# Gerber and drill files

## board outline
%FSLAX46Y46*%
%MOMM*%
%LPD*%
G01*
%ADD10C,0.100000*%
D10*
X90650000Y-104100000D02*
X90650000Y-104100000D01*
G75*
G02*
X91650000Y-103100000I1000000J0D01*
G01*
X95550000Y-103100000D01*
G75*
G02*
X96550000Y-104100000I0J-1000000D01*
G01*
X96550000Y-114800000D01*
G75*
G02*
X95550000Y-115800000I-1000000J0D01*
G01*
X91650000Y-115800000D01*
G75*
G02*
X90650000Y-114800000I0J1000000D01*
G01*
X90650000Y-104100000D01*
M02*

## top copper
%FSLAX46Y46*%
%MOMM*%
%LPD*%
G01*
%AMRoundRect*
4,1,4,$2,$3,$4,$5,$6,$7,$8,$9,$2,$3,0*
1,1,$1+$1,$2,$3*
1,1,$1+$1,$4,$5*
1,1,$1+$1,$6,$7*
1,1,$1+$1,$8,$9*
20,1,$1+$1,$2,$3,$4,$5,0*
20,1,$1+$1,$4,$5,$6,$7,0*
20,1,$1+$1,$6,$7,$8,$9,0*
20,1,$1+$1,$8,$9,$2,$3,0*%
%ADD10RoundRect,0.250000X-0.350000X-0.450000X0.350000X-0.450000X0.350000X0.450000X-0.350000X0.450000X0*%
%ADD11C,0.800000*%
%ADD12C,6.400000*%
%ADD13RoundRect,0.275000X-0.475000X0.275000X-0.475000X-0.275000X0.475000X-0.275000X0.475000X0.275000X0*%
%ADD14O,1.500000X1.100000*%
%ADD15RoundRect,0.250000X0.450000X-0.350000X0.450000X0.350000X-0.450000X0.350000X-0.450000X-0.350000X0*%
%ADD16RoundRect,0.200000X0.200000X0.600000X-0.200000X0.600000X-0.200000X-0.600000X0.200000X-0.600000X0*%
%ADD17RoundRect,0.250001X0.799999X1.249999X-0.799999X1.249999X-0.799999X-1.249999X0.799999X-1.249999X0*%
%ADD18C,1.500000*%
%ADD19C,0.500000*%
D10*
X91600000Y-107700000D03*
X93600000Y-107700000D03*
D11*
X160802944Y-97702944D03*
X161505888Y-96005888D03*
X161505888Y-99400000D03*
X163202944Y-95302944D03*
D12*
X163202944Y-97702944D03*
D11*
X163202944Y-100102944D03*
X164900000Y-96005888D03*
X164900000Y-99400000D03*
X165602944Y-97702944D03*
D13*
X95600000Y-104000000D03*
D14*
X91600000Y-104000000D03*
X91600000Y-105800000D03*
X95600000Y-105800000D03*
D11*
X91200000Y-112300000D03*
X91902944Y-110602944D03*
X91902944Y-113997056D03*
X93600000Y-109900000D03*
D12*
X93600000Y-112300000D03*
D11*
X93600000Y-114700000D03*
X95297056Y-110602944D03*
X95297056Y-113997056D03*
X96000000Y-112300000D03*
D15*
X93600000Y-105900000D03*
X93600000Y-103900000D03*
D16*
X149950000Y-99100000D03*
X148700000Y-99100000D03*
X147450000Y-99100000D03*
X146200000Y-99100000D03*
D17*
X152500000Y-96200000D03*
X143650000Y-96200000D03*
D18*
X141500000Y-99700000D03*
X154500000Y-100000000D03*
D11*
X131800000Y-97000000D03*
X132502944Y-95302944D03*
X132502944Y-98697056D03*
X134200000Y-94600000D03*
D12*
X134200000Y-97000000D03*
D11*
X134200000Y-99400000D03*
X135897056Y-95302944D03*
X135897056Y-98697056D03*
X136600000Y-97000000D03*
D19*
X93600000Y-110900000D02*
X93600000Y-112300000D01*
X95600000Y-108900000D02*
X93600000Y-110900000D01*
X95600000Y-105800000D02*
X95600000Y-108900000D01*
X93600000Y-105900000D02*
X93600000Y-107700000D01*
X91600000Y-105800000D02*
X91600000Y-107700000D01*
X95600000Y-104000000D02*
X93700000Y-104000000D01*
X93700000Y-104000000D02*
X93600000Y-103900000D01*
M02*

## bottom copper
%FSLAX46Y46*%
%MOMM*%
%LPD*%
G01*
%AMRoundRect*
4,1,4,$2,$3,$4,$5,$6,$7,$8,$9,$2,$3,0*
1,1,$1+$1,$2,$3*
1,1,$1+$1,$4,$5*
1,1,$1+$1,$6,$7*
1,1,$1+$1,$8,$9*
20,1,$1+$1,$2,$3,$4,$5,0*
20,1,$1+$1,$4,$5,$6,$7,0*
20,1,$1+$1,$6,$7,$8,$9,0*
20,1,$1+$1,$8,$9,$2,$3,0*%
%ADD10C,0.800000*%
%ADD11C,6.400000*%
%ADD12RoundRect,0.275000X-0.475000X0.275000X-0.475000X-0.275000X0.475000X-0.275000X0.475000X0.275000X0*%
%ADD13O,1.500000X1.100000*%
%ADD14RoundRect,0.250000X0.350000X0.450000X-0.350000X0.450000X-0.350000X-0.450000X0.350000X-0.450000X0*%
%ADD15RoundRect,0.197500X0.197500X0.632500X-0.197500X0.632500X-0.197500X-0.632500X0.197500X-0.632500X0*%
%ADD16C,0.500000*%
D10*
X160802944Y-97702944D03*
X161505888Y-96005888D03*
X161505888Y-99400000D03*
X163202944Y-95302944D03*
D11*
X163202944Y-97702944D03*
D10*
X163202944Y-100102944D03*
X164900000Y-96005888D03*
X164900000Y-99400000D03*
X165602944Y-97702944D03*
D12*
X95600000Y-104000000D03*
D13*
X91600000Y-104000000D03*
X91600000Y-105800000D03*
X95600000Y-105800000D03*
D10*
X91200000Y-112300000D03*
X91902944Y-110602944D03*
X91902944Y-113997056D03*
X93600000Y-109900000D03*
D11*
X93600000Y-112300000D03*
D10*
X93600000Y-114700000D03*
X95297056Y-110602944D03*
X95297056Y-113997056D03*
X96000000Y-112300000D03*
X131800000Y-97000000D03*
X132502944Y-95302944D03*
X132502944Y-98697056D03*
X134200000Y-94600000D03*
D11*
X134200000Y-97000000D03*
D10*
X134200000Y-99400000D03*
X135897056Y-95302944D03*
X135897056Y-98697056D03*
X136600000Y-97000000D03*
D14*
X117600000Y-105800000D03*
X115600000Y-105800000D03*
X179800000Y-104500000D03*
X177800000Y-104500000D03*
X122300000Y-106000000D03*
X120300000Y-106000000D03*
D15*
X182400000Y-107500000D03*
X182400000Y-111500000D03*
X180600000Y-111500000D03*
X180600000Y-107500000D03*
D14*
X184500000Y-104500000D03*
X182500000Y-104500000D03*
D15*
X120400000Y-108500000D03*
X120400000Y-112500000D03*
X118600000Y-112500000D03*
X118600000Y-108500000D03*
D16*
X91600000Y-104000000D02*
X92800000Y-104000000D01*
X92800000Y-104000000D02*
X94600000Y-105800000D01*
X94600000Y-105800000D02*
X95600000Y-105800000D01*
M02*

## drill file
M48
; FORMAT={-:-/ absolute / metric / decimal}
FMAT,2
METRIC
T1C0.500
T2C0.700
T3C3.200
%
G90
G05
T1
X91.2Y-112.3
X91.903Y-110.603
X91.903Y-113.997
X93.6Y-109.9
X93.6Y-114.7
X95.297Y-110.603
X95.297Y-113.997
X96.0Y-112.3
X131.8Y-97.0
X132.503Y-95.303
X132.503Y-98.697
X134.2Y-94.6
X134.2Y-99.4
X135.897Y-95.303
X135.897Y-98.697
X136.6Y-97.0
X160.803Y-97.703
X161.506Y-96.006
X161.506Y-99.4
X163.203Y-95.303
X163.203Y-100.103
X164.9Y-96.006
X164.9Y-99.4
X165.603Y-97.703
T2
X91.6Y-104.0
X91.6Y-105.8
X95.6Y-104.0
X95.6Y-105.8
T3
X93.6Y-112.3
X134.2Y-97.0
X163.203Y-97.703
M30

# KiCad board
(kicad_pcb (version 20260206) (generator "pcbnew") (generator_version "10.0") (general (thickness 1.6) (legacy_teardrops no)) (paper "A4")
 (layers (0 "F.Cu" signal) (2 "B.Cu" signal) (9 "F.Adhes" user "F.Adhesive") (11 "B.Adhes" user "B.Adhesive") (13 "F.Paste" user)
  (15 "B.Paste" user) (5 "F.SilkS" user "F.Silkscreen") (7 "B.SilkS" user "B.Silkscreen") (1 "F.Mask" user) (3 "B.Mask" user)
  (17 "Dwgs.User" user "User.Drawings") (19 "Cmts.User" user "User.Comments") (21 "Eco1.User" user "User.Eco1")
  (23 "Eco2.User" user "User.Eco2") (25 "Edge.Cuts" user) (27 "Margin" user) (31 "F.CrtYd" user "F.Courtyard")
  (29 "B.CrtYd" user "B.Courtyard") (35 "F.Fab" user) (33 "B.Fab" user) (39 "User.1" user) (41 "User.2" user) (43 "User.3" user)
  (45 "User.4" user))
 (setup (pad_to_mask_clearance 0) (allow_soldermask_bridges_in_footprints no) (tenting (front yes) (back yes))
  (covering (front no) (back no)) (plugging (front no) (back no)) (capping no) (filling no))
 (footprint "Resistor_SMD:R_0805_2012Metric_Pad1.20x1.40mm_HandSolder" (layer "F.Cu") (at 92.6 107.7)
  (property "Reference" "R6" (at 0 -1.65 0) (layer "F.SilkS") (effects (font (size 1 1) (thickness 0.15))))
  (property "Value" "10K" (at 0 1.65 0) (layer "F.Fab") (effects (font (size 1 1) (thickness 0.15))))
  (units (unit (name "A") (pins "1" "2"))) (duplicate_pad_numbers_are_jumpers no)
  (pad "1" smd roundrect (at -1 0) (size 1.2 1.4) (layers "F.Cu" "F.Mask" "F.Paste") (roundrect_rratio 0.208333) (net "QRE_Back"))
  (pad "2" smd roundrect (at 1 0) (size 1.2 1.4) (layers "F.Cu" "F.Mask" "F.Paste") (roundrect_rratio 0.208333) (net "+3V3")))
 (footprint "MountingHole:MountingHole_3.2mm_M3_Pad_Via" (layer "F.Cu") (at 163.202944 97.702944)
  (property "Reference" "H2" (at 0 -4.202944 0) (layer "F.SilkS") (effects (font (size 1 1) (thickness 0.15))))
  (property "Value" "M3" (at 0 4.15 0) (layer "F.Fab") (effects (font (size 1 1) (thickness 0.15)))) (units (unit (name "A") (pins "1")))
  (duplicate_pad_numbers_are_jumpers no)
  (pad "1" thru_hole circle (at -2.4 0) (size 0.8 0.8) (drill 0.5) (layers "*.Cu" "*.Mask") (remove_unused_layers no) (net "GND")
   (zone_connect 2))
  (pad "1" thru_hole circle (at -1.697056 -1.697056) (size 0.8 0.8) (drill 0.5) (layers "*.Cu" "*.Mask") (remove_unused_layers no)
   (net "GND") (zone_connect 2))
  (pad "1" thru_hole circle (at -1.697056 1.697056) (size 0.8 0.8) (drill 0.5) (layers "*.Cu" "*.Mask") (remove_unused_layers no)
   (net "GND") (zone_connect 2))
  (pad "1" thru_hole circle (at 0 -2.4) (size 0.8 0.8) (drill 0.5) (layers "*.Cu" "*.Mask") (remove_unused_layers no) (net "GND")
   (zone_connect 2))
  (pad "1" thru_hole circle (at 0 0) (size 6.4 6.4) (drill 3.2) (layers "*.Cu" "*.Mask") (remove_unused_layers no) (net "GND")
   (zone_connect 2))
  (pad "1" thru_hole circle (at 0 2.4) (size 0.8 0.8) (drill 0.5) (layers "*.Cu" "*.Mask") (remove_unused_layers no) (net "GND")
   (zone_connect 2))
  (pad "1" thru_hole circle (at 1.697056 -1.697056) (size 0.8 0.8) (drill 0.5) (layers "*.Cu" "*.Mask") (remove_unused_layers no)
   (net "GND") (zone_connect 2))
  (pad "1" thru_hole circle (at 1.697056 1.697056) (size 0.8 0.8) (drill 0.5) (layers "*.Cu" "*.Mask") (remove_unused_layers no) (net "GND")
   (zone_connect 2))
  (pad "1" thru_hole circle (at 2.4 0) (size 0.8 0.8) (drill 0.5) (layers "*.Cu" "*.Mask") (remove_unused_layers no) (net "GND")
   (zone_connect 2)))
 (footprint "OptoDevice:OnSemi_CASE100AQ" (layer "F.Cu") (at 95.6 104 -90)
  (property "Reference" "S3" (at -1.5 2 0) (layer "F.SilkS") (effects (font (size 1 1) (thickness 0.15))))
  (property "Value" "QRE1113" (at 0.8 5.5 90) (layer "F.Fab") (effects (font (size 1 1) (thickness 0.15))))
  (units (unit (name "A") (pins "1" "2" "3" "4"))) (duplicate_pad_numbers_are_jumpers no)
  (pad "1" thru_hole roundrect (at 0 0 270) (size 1.1 1.5) (drill 0.7) (layers "*.Cu" "*.Mask") (remove_unused_layers no)
   (roundrect_rratio 0.25) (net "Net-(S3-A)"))
  (pad "2" thru_hole oval (at 0 4 270) (size 1.1 1.5) (drill 0.7) (layers "*.Cu" "*.Mask") (remove_unused_layers no) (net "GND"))
  (pad "3" thru_hole oval (at 1.8 4 270) (size 1.1 1.5) (drill 0.7) (layers "*.Cu" "*.Mask") (remove_unused_layers no) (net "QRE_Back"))
  (pad "4" thru_hole oval (at 1.8 0 270) (size 1.1 1.5) (drill 0.7) (layers "*.Cu" "*.Mask") (remove_unused_layers no) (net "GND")))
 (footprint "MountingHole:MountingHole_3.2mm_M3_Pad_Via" (layer "F.Cu") (at 93.6 112.3)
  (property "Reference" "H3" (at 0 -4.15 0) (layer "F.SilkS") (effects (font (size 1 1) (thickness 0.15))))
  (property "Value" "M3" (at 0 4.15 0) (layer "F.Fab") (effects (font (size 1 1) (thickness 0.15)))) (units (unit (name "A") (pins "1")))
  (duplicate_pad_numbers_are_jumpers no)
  (pad "1" thru_hole circle (at -2.4 0) (size 0.8 0.8) (drill 0.5) (layers "*.Cu" "*.Mask") (remove_unused_layers no) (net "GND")
   (zone_connect 2))
  (pad "1" thru_hole circle (at -1.697056 -1.697056) (size 0.8 0.8) (drill 0.5) (layers "*.Cu" "*.Mask") (remove_unused_layers no)
   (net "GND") (zone_connect 2))
  (pad "1" thru_hole circle (at -1.697056 1.697056) (size 0.8 0.8) (drill 0.5) (layers "*.Cu" "*.Mask") (remove_unused_layers no)
   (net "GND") (zone_connect 2))
  (pad "1" thru_hole circle (at 0 -2.4) (size 0.8 0.8) (drill 0.5) (layers "*.Cu" "*.Mask") (remove_unused_layers no) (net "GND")
   (zone_connect 2))
  (pad "1" thru_hole circle (at 0 0) (size 6.4 6.4) (drill 3.2) (layers "*.Cu" "*.Mask") (remove_unused_layers no) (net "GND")
   (zone_connect 2))
  (pad "1" thru_hole circle (at 0 2.4) (size 0.8 0.8) (drill 0.5) (layers "*.Cu" "*.Mask") (remove_unused_layers no) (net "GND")
   (zone_connect 2))
  (pad "1" thru_hole circle (at 1.697056 -1.697056) (size 0.8 0.8) (drill 0.5) (layers "*.Cu" "*.Mask") (remove_unused_layers no)
   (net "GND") (zone_connect 2))
  (pad "1" thru_hole circle (at 1.697056 1.697056) (size 0.8 0.8) (drill 0.5) (layers "*.Cu" "*.Mask") (remove_unused_layers no) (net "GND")
   (zone_connect 2))
  (pad "1" thru_hole circle (at 2.4 0) (size 0.8 0.8) (drill 0.5) (layers "*.Cu" "*.Mask") (remove_unused_layers no) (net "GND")
   (zone_connect 2)))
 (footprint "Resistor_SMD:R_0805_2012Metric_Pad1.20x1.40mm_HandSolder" (layer "F.Cu") (at 93.6 104.9 90)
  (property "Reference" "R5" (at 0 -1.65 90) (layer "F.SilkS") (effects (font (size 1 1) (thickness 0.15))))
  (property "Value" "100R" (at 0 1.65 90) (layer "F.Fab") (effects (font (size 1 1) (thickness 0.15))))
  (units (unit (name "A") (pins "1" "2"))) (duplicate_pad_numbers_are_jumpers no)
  (pad "1" smd roundrect (at -1 0 90) (size 1.2 1.4) (layers "F.Cu" "F.Mask" "F.Paste") (roundrect_rratio 0.208333) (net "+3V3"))
  (pad "2" smd roundrect (at 1 0 90) (size 1.2 1.4) (layers "F.Cu" "F.Mask" "F.Paste") (roundrect_rratio 0.208333) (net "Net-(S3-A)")))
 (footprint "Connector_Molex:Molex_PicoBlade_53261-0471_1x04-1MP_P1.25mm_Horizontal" (layer "F.Cu") (at 148.075 96.7 180)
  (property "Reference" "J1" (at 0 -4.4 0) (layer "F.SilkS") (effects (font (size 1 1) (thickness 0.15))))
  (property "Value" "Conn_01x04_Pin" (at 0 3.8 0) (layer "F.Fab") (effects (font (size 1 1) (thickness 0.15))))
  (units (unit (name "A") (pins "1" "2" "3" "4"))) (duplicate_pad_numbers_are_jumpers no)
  (pad "1" smd roundrect (at -1.875 -2.4 180) (size 0.8 1.6) (layers "F.Cu" "F.Mask" "F.Paste") (roundrect_rratio 0.25) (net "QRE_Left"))
  (pad "2" smd roundrect (at -0.625 -2.4 180) (size 0.8 1.6) (layers "F.Cu" "F.Mask" "F.Paste") (roundrect_rratio 0.25) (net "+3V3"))
  (pad "3" smd roundrect (at 0.625 -2.4 180) (size 0.8 1.6) (layers "F.Cu" "F.Mask" "F.Paste") (roundrect_rratio 0.25) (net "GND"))
  (pad "4" smd roundrect (at 1.875 -2.4 180) (size 0.8 1.6) (layers "F.Cu" "F.Mask" "F.Paste") (roundrect_rratio 0.25) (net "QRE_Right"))
  (pad "MP" smd roundrect (at -4.425 0.5 180) (size 2.1 3) (layers "F.Cu" "F.Mask" "F.Paste") (roundrect_rratio 0.119048))
  (pad "MP" smd roundrect (at 4.425 0.5 180) (size 2.1 3) (layers "F.Cu" "F.Mask" "F.Paste") (roundrect_rratio 0.119048)))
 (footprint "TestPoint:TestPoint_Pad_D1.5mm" (layer "F.Cu") (at 141.5 99.7)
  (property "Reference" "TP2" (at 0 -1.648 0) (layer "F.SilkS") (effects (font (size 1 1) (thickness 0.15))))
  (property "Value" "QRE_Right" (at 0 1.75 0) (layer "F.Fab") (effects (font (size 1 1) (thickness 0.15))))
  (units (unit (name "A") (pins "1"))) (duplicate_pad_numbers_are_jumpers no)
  (pad "1" smd circle (at 0 0) (size 1.5 1.5) (layers "F.Cu" "F.Mask") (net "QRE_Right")))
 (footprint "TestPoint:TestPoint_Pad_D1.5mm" (layer "F.Cu") (at 154.5 100)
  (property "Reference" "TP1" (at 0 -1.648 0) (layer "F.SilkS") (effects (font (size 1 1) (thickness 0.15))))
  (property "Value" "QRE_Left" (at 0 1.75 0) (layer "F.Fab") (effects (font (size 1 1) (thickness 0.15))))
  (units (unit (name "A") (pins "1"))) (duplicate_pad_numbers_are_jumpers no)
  (pad "1" smd circle (at 0 0) (size 1.5 1.5) (layers "F.Cu" "F.Mask") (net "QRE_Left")))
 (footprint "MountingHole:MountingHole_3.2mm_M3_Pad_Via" (layer "F.Cu") (at 134.2 97)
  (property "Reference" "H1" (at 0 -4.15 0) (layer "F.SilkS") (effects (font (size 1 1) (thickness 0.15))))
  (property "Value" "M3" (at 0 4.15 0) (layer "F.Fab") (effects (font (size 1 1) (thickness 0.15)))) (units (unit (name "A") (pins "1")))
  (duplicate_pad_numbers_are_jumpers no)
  (pad "1" thru_hole circle (at -2.4 0) (size 0.8 0.8) (drill 0.5) (layers "*.Cu" "*.Mask") (remove_unused_layers no) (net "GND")
   (zone_connect 2))
  (pad "1" thru_hole circle (at -1.697056 -1.697056) (size 0.8 0.8) (drill 0.5) (layers "*.Cu" "*.Mask") (remove_unused_layers no)
   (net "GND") (zone_connect 2))
  (pad "1" thru_hole circle (at -1.697056 1.697056) (size 0.8 0.8) (drill 0.5) (layers "*.Cu" "*.Mask") (remove_unused_layers no)
   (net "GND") (zone_connect 2))
  (pad "1" thru_hole circle (at 0 -2.4) (size 0.8 0.8) (drill 0.5) (layers "*.Cu" "*.Mask") (remove_unused_layers no) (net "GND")
   (zone_connect 2))
  (pad "1" thru_hole circle (at 0 0) (size 6.4 6.4) (drill 3.2) (layers "*.Cu" "*.Mask") (remove_unused_layers no) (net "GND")
   (zone_connect 2))
  (pad "1" thru_hole circle (at 0 2.4) (size 0.8 0.8) (drill 0.5) (layers "*.Cu" "*.Mask") (remove_unused_layers no) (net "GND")
   (zone_connect 2))
  (pad "1" thru_hole circle (at 1.697056 -1.697056) (size 0.8 0.8) (drill 0.5) (layers "*.Cu" "*.Mask") (remove_unused_layers no)
   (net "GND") (zone_connect 2))
  (pad "1" thru_hole circle (at 1.697056 1.697056) (size 0.8 0.8) (drill 0.5) (layers "*.Cu" "*.Mask") (remove_unused_layers no) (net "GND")
   (zone_connect 2))
  (pad "1" thru_hole circle (at 2.4 0) (size 0.8 0.8) (drill 0.5) (layers "*.Cu" "*.Mask") (remove_unused_layers no) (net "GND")
   (zone_connect 2)))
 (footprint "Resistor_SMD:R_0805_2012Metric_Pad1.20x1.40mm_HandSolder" (layer "B.Cu") (at 116.6 105.8 180)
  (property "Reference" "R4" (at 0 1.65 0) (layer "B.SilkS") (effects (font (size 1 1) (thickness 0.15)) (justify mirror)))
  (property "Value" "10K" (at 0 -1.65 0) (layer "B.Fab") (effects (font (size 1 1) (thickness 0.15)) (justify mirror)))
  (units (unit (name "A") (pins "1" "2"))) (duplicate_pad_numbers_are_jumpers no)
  (pad "1" smd roundrect (at -1 0 180) (size 1.2 1.4) (layers "B.Cu" "B.Mask" "B.Paste") (roundrect_rratio 0.208333) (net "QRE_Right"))
  (pad "2" smd roundrect (at 1 0 180) (size 1.2 1.4) (layers "B.Cu" "B.Mask" "B.Paste") (roundrect_rratio 0.208333) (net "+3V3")))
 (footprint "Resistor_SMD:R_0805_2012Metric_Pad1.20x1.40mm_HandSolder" (layer "B.Cu") (at 178.8 104.5 180)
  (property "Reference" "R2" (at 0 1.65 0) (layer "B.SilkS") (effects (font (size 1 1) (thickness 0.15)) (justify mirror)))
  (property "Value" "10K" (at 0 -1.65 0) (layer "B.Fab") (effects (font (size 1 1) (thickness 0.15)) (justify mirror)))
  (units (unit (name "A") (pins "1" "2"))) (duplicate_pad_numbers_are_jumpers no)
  (pad "1" smd roundrect (at -1 0 180) (size 1.2 1.4) (layers "B.Cu" "B.Mask" "B.Paste") (roundrect_rratio 0.208333) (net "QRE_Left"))
  (pad "2" smd roundrect (at 1 0 180) (size 1.2 1.4) (layers "B.Cu" "B.Mask" "B.Paste") (roundrect_rratio 0.208333) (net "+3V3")))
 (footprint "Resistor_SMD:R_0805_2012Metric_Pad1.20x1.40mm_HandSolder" (layer "B.Cu") (at 121.3 106 180)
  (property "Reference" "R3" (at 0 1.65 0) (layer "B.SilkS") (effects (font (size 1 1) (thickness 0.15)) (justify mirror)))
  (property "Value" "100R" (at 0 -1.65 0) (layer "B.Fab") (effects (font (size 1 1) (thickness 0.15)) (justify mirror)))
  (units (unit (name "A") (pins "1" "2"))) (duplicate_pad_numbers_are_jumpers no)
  (pad "1" smd roundrect (at -1 0 180) (size 1.2 1.4) (layers "B.Cu" "B.Mask" "B.Paste") (roundrect_rratio 0.208333) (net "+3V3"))
  (pad "2" smd roundrect (at 1 0 180) (size 1.2 1.4) (layers "B.Cu" "B.Mask" "B.Paste") (roundrect_rratio 0.208333) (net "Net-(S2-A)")))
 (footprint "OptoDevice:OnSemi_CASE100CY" (layer "B.Cu") (at 181.5 109.5 180)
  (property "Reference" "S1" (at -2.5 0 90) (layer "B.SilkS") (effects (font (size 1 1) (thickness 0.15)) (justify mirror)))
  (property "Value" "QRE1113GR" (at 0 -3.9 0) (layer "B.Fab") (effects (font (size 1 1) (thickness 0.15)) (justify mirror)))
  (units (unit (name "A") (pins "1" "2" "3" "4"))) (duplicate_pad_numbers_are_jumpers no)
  (pad "1" smd roundrect (at -0.9 2 180) (size 0.79 1.66) (layers "B.Cu" "B.Mask" "B.Paste") (roundrect_rratio 0.25) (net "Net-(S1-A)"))
  (pad "2" smd roundrect (at -0.9 -2 180) (size 0.79 1.66) (layers "B.Cu" "B.Mask" "B.Paste") (roundrect_rratio 0.25) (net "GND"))
  (pad "3" smd roundrect (at 0.9 -2 180) (size 0.79 1.66) (layers "B.Cu" "B.Mask" "B.Paste") (roundrect_rratio 0.25) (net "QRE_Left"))
  (pad "4" smd roundrect (at 0.9 2 180) (size 0.79 1.66) (layers "B.Cu" "B.Mask" "B.Paste") (roundrect_rratio 0.25) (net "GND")))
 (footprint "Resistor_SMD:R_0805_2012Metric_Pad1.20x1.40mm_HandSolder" (layer "B.Cu") (at 183.5 104.5 180)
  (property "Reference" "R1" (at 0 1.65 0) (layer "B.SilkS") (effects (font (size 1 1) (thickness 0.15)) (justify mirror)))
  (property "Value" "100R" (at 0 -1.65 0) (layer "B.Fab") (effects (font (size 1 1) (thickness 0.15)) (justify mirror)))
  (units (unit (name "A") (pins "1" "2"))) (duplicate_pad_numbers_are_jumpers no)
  (pad "1" smd roundrect (at -1 0 180) (size 1.2 1.4) (layers "B.Cu" "B.Mask" "B.Paste") (roundrect_rratio 0.208333) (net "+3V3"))
  (pad "2" smd roundrect (at 1 0 180) (size 1.2 1.4) (layers "B.Cu" "B.Mask" "B.Paste") (roundrect_rratio 0.208333) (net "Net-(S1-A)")))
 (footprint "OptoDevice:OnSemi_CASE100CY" (layer "B.Cu") (at 119.5 110.5 180)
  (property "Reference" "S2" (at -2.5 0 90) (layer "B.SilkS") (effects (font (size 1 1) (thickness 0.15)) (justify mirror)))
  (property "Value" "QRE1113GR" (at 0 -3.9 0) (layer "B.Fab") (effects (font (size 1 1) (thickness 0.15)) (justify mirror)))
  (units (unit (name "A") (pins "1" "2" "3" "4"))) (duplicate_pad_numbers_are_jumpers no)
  (pad "1" smd roundrect (at -0.9 2 180) (size 0.79 1.66) (layers "B.Cu" "B.Mask" "B.Paste") (roundrect_rratio 0.25) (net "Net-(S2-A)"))
  (pad "2" smd roundrect (at -0.9 -2 180) (size 0.79 1.66) (layers "B.Cu" "B.Mask" "B.Paste") (roundrect_rratio 0.25) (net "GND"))
  (pad "3" smd roundrect (at 0.9 -2 180) (size 0.79 1.66) (layers "B.Cu" "B.Mask" "B.Paste") (roundrect_rratio 0.25) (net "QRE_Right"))
  (pad "4" smd roundrect (at 0.9 2 180) (size 0.79 1.66) (layers "B.Cu" "B.Mask" "B.Paste") (roundrect_rratio 0.25) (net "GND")))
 (gr_rect (start 90.65 103.1) (end 96.55 115.8) (radius 1) (stroke (width 0.1) (type solid)) (fill no) (layer "Edge.Cuts"))
 (segment (start 93.6 110.9) (end 93.6 112.3) (width 0.5) (layer "F.Cu") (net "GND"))
 (segment (start 95.6 108.9) (end 93.6 110.9) (width 0.5) (layer "F.Cu") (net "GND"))
 (segment (start 95.6 105.8) (end 95.6 108.9) (width 0.5) (layer "F.Cu") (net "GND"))
 (segment (start 91.6 104) (end 92.8 104) (width 0.5) (layer "B.Cu") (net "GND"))
 (segment (start 92.8 104) (end 94.6 105.8) (width 0.5) (layer "B.Cu") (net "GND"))
 (segment (start 94.6 105.8) (end 95.6 105.8) (width 0.5) (layer "B.Cu") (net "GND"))
 (segment (start 93.6 105.9) (end 93.6 107.7) (width 0.5) (layer "F.Cu") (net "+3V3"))
 (segment (start 91.6 105.8) (end 91.6 107.7) (width 0.5) (layer "F.Cu") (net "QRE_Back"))
 (segment (start 95.6 104) (end 93.7 104) (width 0.5) (layer "F.Cu") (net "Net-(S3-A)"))
 (segment (start 93.7 104) (end 93.6 103.9) (width 0.5) (layer "F.Cu") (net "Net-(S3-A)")))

